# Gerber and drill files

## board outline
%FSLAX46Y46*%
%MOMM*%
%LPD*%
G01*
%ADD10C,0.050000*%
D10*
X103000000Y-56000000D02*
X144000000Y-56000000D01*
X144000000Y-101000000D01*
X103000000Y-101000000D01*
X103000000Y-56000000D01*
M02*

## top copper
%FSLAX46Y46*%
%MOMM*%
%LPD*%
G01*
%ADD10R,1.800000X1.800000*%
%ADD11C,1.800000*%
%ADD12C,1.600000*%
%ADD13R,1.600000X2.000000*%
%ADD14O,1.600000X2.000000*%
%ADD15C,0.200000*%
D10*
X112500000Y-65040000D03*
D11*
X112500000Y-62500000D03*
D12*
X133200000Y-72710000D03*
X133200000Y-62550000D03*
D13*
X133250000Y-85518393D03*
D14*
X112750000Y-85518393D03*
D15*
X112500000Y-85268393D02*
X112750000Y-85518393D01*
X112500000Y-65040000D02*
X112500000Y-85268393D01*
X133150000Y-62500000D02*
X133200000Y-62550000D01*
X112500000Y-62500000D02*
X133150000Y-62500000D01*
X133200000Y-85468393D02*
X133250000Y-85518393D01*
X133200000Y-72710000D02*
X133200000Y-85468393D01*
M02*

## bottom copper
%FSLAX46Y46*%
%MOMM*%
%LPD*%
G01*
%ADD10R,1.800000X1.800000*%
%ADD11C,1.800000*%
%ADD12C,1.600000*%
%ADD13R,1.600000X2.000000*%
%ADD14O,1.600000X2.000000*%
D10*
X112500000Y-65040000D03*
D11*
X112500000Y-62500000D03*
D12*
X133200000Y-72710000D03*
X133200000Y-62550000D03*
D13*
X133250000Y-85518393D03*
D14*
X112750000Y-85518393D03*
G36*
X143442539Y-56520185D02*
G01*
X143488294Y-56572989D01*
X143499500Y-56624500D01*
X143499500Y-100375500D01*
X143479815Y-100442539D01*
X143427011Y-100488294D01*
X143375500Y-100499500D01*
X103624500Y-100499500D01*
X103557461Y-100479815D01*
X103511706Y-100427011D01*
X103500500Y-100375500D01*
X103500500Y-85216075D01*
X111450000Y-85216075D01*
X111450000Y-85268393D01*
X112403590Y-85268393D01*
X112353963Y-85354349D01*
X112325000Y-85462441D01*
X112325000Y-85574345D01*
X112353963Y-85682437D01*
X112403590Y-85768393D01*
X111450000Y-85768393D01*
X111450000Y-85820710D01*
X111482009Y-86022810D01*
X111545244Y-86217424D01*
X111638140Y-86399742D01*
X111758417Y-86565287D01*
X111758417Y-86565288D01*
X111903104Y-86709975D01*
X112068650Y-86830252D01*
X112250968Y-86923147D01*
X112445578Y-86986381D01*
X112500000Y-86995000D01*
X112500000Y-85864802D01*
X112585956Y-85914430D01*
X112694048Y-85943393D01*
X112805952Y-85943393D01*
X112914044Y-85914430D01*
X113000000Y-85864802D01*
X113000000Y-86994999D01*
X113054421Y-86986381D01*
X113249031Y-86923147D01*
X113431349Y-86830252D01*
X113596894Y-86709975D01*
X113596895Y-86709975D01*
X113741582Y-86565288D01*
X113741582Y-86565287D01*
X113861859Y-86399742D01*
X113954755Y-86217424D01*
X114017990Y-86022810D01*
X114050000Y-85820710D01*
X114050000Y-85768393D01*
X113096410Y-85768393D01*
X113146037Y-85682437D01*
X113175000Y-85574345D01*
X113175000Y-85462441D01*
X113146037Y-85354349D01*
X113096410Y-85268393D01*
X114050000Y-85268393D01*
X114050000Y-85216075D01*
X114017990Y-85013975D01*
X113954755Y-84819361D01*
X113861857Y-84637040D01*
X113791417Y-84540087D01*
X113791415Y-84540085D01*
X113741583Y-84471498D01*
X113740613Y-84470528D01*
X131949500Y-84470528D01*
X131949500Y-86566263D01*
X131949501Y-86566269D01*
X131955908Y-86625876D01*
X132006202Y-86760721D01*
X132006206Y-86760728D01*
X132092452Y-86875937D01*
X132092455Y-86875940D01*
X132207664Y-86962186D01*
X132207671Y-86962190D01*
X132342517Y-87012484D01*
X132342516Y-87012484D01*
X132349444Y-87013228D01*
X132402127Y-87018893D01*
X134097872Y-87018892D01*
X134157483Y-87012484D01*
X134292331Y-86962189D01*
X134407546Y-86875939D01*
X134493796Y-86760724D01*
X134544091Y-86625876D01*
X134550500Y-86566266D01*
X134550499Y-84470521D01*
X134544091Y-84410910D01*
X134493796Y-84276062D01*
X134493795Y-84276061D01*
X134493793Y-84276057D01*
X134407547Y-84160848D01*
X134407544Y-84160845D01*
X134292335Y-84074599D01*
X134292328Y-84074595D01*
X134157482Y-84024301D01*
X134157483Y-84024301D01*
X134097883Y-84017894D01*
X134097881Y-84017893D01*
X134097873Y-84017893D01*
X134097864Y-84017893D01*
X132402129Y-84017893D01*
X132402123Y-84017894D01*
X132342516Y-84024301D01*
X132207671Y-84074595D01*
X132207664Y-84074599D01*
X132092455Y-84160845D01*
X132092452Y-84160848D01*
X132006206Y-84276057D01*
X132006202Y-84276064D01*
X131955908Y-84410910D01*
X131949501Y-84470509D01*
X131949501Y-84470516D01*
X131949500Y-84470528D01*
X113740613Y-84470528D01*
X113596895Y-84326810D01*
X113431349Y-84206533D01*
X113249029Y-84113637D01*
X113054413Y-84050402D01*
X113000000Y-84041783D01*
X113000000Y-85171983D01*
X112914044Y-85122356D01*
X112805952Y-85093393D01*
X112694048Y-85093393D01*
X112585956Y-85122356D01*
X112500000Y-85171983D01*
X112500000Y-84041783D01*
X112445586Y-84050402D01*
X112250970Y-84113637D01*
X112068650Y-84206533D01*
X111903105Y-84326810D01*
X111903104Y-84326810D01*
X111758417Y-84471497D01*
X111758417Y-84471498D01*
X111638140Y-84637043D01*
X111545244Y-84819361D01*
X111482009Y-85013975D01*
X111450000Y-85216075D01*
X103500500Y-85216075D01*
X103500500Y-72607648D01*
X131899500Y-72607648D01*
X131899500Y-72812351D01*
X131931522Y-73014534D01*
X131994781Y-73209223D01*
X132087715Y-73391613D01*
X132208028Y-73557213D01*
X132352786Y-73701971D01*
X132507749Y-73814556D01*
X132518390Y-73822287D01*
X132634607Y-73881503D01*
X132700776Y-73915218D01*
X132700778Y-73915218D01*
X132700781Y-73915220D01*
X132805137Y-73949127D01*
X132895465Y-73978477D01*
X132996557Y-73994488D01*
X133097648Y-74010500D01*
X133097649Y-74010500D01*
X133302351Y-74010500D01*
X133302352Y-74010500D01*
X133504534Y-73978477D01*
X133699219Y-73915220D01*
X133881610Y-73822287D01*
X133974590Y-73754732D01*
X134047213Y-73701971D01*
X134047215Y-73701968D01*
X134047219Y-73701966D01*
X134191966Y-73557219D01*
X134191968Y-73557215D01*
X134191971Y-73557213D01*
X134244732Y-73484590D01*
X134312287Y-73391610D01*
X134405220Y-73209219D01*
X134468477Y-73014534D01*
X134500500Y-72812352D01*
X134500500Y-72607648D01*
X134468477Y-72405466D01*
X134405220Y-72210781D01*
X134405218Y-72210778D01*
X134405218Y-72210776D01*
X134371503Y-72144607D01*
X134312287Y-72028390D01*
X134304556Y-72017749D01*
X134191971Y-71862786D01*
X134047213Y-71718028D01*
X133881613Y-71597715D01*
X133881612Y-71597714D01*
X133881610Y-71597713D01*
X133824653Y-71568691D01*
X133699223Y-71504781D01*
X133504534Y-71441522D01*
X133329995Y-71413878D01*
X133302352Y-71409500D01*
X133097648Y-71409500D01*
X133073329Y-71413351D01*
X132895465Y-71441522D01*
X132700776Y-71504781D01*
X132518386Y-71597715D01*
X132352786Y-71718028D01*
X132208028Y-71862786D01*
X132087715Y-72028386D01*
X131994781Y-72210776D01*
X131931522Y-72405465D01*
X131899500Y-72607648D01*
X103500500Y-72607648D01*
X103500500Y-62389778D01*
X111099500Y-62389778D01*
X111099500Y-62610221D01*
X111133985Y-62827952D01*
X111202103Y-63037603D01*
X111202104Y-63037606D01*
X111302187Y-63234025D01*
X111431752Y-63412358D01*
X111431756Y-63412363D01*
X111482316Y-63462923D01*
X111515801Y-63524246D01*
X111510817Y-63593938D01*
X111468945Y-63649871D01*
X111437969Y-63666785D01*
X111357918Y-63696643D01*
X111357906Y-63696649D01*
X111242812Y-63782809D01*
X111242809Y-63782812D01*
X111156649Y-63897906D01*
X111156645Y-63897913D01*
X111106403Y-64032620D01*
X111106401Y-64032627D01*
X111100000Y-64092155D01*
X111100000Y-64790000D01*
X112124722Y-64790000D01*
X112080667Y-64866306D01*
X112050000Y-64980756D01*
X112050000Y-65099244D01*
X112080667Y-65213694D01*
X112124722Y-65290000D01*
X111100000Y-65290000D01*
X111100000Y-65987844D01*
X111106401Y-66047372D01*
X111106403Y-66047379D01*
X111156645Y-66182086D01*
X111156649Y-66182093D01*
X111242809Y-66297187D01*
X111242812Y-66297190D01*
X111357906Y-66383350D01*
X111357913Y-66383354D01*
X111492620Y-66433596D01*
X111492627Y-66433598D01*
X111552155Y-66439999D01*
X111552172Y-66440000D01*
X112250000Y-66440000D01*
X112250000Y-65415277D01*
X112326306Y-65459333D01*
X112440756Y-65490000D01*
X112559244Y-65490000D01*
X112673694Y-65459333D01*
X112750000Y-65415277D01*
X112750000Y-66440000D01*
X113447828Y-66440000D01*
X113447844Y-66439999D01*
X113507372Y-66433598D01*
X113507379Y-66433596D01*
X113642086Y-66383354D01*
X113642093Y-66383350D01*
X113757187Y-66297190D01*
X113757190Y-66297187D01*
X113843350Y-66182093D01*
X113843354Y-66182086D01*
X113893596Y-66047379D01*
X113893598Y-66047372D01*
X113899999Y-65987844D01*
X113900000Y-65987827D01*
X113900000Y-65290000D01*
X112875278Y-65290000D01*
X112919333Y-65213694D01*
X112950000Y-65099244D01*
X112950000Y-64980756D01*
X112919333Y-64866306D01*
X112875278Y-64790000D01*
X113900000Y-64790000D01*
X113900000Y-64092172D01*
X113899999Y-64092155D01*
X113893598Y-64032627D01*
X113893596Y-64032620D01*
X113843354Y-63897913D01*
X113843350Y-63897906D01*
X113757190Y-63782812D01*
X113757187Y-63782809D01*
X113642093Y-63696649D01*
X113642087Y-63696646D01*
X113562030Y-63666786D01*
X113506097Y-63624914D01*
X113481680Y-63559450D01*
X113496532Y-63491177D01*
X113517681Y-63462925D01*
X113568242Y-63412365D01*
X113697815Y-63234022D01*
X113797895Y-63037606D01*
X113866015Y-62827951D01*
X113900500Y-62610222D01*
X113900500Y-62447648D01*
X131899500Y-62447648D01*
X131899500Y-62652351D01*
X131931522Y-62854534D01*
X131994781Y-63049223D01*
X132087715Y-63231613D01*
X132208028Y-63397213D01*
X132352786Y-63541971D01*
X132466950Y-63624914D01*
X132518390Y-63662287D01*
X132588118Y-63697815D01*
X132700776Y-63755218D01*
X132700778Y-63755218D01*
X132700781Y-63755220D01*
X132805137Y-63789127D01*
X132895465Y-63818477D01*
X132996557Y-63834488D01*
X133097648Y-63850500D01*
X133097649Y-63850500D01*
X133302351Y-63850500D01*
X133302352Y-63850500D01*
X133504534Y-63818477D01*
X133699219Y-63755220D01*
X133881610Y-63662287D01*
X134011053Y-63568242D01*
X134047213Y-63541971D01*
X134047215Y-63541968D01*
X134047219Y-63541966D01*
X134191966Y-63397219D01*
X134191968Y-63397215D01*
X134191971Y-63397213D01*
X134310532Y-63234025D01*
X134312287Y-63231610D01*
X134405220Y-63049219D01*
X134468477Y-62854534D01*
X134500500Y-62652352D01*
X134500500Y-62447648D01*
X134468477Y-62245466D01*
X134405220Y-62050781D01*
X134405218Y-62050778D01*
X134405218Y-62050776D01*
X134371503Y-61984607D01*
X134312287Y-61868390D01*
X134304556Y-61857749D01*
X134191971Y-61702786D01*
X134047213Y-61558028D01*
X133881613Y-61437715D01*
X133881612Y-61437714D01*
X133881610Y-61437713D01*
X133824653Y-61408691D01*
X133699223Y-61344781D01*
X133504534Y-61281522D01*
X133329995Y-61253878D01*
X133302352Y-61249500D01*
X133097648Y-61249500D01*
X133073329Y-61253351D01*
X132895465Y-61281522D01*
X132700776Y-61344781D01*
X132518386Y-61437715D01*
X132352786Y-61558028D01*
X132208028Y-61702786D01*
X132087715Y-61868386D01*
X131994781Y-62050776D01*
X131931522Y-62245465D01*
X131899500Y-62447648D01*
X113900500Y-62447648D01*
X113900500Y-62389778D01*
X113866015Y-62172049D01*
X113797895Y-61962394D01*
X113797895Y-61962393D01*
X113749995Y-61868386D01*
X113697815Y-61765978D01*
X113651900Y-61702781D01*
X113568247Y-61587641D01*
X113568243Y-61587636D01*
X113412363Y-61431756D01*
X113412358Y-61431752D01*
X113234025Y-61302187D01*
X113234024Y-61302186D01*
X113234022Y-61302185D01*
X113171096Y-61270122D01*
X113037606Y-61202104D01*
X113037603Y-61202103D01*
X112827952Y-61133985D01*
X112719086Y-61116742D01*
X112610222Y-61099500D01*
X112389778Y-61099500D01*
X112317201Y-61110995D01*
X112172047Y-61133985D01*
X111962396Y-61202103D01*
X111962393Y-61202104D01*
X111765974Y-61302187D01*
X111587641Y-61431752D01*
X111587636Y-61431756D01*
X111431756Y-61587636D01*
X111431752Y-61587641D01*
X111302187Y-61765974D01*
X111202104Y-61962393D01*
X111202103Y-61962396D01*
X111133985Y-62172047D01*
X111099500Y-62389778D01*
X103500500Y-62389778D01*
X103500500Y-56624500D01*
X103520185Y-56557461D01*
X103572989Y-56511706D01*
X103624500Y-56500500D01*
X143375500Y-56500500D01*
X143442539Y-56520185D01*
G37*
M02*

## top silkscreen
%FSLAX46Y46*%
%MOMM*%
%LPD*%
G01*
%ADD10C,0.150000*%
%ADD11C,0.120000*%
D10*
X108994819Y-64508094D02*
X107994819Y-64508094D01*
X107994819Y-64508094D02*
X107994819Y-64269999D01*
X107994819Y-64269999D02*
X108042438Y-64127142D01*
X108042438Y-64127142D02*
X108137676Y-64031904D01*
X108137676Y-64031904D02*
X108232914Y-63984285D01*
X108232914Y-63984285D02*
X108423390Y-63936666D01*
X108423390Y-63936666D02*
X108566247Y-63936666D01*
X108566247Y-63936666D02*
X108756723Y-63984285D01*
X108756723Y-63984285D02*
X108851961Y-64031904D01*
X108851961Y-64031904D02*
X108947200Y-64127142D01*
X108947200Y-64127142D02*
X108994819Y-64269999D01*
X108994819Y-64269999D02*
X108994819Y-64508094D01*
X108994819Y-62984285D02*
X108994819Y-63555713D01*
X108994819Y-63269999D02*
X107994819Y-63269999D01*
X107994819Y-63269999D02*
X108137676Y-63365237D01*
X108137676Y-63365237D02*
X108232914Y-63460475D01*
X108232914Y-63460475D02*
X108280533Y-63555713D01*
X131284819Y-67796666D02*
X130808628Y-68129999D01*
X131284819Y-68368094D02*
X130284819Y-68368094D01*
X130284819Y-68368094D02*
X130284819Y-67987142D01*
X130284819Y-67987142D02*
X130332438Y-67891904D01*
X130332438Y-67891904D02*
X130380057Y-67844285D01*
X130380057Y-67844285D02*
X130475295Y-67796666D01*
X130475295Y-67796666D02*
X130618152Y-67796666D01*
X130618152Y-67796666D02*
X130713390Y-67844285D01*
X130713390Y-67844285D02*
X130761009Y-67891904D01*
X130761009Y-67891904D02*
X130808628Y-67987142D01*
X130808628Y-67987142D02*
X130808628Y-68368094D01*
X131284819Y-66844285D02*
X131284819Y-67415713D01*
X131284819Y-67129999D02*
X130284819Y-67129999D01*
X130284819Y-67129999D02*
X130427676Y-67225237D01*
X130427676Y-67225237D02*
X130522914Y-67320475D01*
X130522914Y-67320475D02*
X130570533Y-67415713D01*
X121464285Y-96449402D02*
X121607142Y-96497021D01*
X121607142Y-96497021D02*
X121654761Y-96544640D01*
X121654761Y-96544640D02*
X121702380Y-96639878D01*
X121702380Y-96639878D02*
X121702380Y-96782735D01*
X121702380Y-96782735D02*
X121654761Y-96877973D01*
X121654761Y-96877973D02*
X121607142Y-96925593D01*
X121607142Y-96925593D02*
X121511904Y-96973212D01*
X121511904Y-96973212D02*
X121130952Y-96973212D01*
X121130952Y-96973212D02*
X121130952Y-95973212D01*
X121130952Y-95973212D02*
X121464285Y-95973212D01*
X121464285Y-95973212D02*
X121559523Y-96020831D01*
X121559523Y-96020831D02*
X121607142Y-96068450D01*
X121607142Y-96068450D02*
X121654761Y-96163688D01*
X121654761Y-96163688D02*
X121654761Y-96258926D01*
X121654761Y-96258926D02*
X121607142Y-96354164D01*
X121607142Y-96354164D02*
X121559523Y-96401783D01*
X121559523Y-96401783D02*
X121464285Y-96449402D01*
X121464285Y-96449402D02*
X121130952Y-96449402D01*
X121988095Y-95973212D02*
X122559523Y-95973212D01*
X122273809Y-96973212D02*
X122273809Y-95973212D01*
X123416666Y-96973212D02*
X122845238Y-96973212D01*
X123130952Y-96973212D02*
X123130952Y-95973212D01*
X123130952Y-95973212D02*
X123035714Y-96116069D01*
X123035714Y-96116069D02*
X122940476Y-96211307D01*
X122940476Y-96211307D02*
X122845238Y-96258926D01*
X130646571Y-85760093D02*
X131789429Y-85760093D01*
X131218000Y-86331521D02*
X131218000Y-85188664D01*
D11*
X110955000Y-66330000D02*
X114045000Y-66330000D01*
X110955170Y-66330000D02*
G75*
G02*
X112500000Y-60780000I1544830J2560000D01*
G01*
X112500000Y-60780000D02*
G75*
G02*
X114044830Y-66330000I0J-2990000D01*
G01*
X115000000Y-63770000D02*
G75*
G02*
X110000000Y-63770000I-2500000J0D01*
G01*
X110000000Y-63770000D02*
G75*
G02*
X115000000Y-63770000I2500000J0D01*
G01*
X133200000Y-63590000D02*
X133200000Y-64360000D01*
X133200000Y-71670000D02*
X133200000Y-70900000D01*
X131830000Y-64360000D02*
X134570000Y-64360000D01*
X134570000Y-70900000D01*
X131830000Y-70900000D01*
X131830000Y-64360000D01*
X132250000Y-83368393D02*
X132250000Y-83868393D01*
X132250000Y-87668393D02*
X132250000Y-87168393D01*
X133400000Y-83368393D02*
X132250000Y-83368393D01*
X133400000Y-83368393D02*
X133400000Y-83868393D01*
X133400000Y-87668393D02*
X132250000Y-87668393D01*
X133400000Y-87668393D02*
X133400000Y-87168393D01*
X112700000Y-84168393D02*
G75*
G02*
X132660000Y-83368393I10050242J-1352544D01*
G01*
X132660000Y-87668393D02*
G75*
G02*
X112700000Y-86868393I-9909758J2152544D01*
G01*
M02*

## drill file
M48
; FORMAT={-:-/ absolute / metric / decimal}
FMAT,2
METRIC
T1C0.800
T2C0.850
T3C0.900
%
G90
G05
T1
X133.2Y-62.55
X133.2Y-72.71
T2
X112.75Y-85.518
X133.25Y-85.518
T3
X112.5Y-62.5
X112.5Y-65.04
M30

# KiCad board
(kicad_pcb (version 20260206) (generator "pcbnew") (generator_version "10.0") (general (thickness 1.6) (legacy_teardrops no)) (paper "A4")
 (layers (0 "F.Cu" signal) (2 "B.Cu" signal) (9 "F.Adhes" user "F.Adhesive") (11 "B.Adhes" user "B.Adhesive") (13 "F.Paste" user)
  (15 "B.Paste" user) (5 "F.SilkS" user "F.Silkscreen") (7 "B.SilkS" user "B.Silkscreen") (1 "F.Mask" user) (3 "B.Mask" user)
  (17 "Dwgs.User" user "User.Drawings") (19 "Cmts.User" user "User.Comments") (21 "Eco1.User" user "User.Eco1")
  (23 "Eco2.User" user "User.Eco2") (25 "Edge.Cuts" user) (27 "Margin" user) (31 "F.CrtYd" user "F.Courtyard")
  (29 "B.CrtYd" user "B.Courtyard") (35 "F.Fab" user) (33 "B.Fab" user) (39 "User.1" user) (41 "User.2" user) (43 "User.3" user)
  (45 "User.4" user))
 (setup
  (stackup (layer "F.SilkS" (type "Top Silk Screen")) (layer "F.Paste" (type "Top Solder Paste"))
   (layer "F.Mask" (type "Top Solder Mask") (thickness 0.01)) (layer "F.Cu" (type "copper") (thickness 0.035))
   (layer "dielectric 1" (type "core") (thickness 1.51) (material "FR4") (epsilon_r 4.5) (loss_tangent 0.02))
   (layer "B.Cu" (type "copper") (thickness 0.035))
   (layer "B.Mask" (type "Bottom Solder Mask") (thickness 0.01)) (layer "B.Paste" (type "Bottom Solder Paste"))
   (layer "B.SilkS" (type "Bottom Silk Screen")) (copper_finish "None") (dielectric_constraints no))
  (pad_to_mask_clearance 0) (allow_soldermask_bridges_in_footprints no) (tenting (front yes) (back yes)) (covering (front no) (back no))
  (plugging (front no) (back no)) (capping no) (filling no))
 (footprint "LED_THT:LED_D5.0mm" (layer "F.Cu") (at 112.5 65.04 90)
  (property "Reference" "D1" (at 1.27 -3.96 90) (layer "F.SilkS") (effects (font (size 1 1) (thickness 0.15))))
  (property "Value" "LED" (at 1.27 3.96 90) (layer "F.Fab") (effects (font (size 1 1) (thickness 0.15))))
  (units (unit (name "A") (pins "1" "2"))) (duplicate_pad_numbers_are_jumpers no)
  (fp_line (start -1.29 -1.545) (end -1.29 1.545) (stroke (width 0.12) (type solid)) (layer "F.SilkS"))
  (fp_arc (start -1.29 -1.54483) (mid 2.071779 -2.880495) (end 4.26 0) (stroke (width 0.12) (type solid)) (layer "F.SilkS"))
  (fp_arc (start 4.26 0) (mid 2.071779 2.880495) (end -1.29 1.54483) (stroke (width 0.12) (type solid)) (layer "F.SilkS"))
  (fp_circle (center 1.27 0) (end 3.77 0) (stroke (width 0.12) (type solid)) (fill no) (layer "F.SilkS"))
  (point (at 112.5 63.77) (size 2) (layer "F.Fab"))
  (pad "1" thru_hole rect (at 0 0 90) (size 1.8 1.8) (drill 0.9) (layers "*.Cu" "*.Mask") (remove_unused_layers no) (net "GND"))
  (pad "2" thru_hole circle (at 2.54 0 90) (size 1.8 1.8) (drill 0.9) (layers "*.Cu" "*.Mask") (remove_unused_layers no) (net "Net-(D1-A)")))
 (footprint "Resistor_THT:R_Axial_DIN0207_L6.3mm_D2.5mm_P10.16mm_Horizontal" (layer "F.Cu") (at 133.2 72.71 90)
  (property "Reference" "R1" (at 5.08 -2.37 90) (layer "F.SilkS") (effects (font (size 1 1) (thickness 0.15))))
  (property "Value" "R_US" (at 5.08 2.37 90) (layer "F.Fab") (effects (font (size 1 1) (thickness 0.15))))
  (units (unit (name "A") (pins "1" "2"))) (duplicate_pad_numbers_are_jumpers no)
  (fp_line (start 9.12 0) (end 8.35 0) (stroke (width 0.12) (type solid)) (layer "F.SilkS"))
  (fp_line (start 1.04 0) (end 1.81 0) (stroke (width 0.12) (type solid)) (layer "F.SilkS"))
  (fp_rect (start 1.81 -1.37) (end 8.35 1.37) (stroke (width 0.12) (type solid)) (fill no) (layer "F.SilkS"))
  (pad "1" thru_hole circle (at 0 0 90) (size 1.6 1.6) (drill 0.8) (layers "*.Cu" "*.Mask") (remove_unused_layers no) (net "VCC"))
  (pad "2" thru_hole circle (at 10.16 0 90) (size 1.6 1.6) (drill 0.8) (layers "*.Cu" "*.Mask") (remove_unused_layers no) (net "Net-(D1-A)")))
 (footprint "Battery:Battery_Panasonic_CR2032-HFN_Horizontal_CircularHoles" (layer "F.Cu") (at 133.25 85.518393 180)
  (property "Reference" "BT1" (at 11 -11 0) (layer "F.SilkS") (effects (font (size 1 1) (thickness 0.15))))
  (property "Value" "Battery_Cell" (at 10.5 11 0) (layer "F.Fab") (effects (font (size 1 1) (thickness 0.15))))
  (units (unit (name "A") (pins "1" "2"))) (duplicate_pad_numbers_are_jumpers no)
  (fp_line (start 1 2.15) (end 1 1.65) (stroke (width 0.12) (type default)) (layer "F.SilkS"))
  (fp_line (start 1 -2.15) (end 1 -1.65) (stroke (width 0.12) (type default)) (layer "F.SilkS"))
  (fp_line (start -0.15 2.15) (end 1 2.15) (stroke (width 0.12) (type default)) (layer "F.SilkS"))
  (fp_line (start -0.15 2.15) (end -0.15 1.65) (stroke (width 0.12) (type default)) (layer "F.SilkS"))
  (fp_line (start -0.15 -2.15) (end 1 -2.15) (stroke (width 0.12) (type default)) (layer "F.SilkS"))
  (fp_line (start -0.15 -2.15) (end -0.15 -1.65) (stroke (width 0.12) (type default)) (layer "F.SilkS"))
  (fp_arc (start 20.55 1.35) (mid 10.91 10.13) (end 0.59 2.15) (stroke (width 0.12) (type default)) (layer "F.SilkS"))
  (fp_arc (start 0.59 -2.15) (mid 10.91 -10.13) (end 20.55 -1.35) (stroke (width 0.12) (type default)) (layer "F.SilkS"))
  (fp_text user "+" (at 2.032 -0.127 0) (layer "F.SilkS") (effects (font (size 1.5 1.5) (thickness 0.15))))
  (pad "1" thru_hole rect (at 0 0 180) (size 1.6 2) (drill 0.85) (layers "*.Cu" "*.Mask") (remove_unused_layers no) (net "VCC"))
  (pad "2" thru_hole oval (at 20.5 0 180) (size 1.6 2) (drill 0.85) (layers "*.Cu" "*.Mask") (remove_unused_layers no) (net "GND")))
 (gr_rect (start 103 56) (end 144 101) (stroke (width 0.05) (type default)) (fill no) (layer "Edge.Cuts"))
 (segment (start 112.5 85.268393) (end 112.75 85.518393) (width 0.2) (layer "F.Cu") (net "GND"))
 (segment (start 112.5 65.04) (end 112.5 85.268393) (width 0.2) (layer "F.Cu") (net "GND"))
 (segment (start 133.15 62.5) (end 133.2 62.55) (width 0.2) (layer "F.Cu") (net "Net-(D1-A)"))
 (segment (start 112.5 62.5) (end 133.15 62.5) (width 0.2) (layer "F.Cu") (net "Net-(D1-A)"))
 (segment (start 133.2 85.468393) (end 133.25 85.518393) (width 0.2) (layer "F.Cu") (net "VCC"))
 (segment (start 133.2 72.71) (end 133.2 85.468393) (width 0.2) (layer "F.Cu") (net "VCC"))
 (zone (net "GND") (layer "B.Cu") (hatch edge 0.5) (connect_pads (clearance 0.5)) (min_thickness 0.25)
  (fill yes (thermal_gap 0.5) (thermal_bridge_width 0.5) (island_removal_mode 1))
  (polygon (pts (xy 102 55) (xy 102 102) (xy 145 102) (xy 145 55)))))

